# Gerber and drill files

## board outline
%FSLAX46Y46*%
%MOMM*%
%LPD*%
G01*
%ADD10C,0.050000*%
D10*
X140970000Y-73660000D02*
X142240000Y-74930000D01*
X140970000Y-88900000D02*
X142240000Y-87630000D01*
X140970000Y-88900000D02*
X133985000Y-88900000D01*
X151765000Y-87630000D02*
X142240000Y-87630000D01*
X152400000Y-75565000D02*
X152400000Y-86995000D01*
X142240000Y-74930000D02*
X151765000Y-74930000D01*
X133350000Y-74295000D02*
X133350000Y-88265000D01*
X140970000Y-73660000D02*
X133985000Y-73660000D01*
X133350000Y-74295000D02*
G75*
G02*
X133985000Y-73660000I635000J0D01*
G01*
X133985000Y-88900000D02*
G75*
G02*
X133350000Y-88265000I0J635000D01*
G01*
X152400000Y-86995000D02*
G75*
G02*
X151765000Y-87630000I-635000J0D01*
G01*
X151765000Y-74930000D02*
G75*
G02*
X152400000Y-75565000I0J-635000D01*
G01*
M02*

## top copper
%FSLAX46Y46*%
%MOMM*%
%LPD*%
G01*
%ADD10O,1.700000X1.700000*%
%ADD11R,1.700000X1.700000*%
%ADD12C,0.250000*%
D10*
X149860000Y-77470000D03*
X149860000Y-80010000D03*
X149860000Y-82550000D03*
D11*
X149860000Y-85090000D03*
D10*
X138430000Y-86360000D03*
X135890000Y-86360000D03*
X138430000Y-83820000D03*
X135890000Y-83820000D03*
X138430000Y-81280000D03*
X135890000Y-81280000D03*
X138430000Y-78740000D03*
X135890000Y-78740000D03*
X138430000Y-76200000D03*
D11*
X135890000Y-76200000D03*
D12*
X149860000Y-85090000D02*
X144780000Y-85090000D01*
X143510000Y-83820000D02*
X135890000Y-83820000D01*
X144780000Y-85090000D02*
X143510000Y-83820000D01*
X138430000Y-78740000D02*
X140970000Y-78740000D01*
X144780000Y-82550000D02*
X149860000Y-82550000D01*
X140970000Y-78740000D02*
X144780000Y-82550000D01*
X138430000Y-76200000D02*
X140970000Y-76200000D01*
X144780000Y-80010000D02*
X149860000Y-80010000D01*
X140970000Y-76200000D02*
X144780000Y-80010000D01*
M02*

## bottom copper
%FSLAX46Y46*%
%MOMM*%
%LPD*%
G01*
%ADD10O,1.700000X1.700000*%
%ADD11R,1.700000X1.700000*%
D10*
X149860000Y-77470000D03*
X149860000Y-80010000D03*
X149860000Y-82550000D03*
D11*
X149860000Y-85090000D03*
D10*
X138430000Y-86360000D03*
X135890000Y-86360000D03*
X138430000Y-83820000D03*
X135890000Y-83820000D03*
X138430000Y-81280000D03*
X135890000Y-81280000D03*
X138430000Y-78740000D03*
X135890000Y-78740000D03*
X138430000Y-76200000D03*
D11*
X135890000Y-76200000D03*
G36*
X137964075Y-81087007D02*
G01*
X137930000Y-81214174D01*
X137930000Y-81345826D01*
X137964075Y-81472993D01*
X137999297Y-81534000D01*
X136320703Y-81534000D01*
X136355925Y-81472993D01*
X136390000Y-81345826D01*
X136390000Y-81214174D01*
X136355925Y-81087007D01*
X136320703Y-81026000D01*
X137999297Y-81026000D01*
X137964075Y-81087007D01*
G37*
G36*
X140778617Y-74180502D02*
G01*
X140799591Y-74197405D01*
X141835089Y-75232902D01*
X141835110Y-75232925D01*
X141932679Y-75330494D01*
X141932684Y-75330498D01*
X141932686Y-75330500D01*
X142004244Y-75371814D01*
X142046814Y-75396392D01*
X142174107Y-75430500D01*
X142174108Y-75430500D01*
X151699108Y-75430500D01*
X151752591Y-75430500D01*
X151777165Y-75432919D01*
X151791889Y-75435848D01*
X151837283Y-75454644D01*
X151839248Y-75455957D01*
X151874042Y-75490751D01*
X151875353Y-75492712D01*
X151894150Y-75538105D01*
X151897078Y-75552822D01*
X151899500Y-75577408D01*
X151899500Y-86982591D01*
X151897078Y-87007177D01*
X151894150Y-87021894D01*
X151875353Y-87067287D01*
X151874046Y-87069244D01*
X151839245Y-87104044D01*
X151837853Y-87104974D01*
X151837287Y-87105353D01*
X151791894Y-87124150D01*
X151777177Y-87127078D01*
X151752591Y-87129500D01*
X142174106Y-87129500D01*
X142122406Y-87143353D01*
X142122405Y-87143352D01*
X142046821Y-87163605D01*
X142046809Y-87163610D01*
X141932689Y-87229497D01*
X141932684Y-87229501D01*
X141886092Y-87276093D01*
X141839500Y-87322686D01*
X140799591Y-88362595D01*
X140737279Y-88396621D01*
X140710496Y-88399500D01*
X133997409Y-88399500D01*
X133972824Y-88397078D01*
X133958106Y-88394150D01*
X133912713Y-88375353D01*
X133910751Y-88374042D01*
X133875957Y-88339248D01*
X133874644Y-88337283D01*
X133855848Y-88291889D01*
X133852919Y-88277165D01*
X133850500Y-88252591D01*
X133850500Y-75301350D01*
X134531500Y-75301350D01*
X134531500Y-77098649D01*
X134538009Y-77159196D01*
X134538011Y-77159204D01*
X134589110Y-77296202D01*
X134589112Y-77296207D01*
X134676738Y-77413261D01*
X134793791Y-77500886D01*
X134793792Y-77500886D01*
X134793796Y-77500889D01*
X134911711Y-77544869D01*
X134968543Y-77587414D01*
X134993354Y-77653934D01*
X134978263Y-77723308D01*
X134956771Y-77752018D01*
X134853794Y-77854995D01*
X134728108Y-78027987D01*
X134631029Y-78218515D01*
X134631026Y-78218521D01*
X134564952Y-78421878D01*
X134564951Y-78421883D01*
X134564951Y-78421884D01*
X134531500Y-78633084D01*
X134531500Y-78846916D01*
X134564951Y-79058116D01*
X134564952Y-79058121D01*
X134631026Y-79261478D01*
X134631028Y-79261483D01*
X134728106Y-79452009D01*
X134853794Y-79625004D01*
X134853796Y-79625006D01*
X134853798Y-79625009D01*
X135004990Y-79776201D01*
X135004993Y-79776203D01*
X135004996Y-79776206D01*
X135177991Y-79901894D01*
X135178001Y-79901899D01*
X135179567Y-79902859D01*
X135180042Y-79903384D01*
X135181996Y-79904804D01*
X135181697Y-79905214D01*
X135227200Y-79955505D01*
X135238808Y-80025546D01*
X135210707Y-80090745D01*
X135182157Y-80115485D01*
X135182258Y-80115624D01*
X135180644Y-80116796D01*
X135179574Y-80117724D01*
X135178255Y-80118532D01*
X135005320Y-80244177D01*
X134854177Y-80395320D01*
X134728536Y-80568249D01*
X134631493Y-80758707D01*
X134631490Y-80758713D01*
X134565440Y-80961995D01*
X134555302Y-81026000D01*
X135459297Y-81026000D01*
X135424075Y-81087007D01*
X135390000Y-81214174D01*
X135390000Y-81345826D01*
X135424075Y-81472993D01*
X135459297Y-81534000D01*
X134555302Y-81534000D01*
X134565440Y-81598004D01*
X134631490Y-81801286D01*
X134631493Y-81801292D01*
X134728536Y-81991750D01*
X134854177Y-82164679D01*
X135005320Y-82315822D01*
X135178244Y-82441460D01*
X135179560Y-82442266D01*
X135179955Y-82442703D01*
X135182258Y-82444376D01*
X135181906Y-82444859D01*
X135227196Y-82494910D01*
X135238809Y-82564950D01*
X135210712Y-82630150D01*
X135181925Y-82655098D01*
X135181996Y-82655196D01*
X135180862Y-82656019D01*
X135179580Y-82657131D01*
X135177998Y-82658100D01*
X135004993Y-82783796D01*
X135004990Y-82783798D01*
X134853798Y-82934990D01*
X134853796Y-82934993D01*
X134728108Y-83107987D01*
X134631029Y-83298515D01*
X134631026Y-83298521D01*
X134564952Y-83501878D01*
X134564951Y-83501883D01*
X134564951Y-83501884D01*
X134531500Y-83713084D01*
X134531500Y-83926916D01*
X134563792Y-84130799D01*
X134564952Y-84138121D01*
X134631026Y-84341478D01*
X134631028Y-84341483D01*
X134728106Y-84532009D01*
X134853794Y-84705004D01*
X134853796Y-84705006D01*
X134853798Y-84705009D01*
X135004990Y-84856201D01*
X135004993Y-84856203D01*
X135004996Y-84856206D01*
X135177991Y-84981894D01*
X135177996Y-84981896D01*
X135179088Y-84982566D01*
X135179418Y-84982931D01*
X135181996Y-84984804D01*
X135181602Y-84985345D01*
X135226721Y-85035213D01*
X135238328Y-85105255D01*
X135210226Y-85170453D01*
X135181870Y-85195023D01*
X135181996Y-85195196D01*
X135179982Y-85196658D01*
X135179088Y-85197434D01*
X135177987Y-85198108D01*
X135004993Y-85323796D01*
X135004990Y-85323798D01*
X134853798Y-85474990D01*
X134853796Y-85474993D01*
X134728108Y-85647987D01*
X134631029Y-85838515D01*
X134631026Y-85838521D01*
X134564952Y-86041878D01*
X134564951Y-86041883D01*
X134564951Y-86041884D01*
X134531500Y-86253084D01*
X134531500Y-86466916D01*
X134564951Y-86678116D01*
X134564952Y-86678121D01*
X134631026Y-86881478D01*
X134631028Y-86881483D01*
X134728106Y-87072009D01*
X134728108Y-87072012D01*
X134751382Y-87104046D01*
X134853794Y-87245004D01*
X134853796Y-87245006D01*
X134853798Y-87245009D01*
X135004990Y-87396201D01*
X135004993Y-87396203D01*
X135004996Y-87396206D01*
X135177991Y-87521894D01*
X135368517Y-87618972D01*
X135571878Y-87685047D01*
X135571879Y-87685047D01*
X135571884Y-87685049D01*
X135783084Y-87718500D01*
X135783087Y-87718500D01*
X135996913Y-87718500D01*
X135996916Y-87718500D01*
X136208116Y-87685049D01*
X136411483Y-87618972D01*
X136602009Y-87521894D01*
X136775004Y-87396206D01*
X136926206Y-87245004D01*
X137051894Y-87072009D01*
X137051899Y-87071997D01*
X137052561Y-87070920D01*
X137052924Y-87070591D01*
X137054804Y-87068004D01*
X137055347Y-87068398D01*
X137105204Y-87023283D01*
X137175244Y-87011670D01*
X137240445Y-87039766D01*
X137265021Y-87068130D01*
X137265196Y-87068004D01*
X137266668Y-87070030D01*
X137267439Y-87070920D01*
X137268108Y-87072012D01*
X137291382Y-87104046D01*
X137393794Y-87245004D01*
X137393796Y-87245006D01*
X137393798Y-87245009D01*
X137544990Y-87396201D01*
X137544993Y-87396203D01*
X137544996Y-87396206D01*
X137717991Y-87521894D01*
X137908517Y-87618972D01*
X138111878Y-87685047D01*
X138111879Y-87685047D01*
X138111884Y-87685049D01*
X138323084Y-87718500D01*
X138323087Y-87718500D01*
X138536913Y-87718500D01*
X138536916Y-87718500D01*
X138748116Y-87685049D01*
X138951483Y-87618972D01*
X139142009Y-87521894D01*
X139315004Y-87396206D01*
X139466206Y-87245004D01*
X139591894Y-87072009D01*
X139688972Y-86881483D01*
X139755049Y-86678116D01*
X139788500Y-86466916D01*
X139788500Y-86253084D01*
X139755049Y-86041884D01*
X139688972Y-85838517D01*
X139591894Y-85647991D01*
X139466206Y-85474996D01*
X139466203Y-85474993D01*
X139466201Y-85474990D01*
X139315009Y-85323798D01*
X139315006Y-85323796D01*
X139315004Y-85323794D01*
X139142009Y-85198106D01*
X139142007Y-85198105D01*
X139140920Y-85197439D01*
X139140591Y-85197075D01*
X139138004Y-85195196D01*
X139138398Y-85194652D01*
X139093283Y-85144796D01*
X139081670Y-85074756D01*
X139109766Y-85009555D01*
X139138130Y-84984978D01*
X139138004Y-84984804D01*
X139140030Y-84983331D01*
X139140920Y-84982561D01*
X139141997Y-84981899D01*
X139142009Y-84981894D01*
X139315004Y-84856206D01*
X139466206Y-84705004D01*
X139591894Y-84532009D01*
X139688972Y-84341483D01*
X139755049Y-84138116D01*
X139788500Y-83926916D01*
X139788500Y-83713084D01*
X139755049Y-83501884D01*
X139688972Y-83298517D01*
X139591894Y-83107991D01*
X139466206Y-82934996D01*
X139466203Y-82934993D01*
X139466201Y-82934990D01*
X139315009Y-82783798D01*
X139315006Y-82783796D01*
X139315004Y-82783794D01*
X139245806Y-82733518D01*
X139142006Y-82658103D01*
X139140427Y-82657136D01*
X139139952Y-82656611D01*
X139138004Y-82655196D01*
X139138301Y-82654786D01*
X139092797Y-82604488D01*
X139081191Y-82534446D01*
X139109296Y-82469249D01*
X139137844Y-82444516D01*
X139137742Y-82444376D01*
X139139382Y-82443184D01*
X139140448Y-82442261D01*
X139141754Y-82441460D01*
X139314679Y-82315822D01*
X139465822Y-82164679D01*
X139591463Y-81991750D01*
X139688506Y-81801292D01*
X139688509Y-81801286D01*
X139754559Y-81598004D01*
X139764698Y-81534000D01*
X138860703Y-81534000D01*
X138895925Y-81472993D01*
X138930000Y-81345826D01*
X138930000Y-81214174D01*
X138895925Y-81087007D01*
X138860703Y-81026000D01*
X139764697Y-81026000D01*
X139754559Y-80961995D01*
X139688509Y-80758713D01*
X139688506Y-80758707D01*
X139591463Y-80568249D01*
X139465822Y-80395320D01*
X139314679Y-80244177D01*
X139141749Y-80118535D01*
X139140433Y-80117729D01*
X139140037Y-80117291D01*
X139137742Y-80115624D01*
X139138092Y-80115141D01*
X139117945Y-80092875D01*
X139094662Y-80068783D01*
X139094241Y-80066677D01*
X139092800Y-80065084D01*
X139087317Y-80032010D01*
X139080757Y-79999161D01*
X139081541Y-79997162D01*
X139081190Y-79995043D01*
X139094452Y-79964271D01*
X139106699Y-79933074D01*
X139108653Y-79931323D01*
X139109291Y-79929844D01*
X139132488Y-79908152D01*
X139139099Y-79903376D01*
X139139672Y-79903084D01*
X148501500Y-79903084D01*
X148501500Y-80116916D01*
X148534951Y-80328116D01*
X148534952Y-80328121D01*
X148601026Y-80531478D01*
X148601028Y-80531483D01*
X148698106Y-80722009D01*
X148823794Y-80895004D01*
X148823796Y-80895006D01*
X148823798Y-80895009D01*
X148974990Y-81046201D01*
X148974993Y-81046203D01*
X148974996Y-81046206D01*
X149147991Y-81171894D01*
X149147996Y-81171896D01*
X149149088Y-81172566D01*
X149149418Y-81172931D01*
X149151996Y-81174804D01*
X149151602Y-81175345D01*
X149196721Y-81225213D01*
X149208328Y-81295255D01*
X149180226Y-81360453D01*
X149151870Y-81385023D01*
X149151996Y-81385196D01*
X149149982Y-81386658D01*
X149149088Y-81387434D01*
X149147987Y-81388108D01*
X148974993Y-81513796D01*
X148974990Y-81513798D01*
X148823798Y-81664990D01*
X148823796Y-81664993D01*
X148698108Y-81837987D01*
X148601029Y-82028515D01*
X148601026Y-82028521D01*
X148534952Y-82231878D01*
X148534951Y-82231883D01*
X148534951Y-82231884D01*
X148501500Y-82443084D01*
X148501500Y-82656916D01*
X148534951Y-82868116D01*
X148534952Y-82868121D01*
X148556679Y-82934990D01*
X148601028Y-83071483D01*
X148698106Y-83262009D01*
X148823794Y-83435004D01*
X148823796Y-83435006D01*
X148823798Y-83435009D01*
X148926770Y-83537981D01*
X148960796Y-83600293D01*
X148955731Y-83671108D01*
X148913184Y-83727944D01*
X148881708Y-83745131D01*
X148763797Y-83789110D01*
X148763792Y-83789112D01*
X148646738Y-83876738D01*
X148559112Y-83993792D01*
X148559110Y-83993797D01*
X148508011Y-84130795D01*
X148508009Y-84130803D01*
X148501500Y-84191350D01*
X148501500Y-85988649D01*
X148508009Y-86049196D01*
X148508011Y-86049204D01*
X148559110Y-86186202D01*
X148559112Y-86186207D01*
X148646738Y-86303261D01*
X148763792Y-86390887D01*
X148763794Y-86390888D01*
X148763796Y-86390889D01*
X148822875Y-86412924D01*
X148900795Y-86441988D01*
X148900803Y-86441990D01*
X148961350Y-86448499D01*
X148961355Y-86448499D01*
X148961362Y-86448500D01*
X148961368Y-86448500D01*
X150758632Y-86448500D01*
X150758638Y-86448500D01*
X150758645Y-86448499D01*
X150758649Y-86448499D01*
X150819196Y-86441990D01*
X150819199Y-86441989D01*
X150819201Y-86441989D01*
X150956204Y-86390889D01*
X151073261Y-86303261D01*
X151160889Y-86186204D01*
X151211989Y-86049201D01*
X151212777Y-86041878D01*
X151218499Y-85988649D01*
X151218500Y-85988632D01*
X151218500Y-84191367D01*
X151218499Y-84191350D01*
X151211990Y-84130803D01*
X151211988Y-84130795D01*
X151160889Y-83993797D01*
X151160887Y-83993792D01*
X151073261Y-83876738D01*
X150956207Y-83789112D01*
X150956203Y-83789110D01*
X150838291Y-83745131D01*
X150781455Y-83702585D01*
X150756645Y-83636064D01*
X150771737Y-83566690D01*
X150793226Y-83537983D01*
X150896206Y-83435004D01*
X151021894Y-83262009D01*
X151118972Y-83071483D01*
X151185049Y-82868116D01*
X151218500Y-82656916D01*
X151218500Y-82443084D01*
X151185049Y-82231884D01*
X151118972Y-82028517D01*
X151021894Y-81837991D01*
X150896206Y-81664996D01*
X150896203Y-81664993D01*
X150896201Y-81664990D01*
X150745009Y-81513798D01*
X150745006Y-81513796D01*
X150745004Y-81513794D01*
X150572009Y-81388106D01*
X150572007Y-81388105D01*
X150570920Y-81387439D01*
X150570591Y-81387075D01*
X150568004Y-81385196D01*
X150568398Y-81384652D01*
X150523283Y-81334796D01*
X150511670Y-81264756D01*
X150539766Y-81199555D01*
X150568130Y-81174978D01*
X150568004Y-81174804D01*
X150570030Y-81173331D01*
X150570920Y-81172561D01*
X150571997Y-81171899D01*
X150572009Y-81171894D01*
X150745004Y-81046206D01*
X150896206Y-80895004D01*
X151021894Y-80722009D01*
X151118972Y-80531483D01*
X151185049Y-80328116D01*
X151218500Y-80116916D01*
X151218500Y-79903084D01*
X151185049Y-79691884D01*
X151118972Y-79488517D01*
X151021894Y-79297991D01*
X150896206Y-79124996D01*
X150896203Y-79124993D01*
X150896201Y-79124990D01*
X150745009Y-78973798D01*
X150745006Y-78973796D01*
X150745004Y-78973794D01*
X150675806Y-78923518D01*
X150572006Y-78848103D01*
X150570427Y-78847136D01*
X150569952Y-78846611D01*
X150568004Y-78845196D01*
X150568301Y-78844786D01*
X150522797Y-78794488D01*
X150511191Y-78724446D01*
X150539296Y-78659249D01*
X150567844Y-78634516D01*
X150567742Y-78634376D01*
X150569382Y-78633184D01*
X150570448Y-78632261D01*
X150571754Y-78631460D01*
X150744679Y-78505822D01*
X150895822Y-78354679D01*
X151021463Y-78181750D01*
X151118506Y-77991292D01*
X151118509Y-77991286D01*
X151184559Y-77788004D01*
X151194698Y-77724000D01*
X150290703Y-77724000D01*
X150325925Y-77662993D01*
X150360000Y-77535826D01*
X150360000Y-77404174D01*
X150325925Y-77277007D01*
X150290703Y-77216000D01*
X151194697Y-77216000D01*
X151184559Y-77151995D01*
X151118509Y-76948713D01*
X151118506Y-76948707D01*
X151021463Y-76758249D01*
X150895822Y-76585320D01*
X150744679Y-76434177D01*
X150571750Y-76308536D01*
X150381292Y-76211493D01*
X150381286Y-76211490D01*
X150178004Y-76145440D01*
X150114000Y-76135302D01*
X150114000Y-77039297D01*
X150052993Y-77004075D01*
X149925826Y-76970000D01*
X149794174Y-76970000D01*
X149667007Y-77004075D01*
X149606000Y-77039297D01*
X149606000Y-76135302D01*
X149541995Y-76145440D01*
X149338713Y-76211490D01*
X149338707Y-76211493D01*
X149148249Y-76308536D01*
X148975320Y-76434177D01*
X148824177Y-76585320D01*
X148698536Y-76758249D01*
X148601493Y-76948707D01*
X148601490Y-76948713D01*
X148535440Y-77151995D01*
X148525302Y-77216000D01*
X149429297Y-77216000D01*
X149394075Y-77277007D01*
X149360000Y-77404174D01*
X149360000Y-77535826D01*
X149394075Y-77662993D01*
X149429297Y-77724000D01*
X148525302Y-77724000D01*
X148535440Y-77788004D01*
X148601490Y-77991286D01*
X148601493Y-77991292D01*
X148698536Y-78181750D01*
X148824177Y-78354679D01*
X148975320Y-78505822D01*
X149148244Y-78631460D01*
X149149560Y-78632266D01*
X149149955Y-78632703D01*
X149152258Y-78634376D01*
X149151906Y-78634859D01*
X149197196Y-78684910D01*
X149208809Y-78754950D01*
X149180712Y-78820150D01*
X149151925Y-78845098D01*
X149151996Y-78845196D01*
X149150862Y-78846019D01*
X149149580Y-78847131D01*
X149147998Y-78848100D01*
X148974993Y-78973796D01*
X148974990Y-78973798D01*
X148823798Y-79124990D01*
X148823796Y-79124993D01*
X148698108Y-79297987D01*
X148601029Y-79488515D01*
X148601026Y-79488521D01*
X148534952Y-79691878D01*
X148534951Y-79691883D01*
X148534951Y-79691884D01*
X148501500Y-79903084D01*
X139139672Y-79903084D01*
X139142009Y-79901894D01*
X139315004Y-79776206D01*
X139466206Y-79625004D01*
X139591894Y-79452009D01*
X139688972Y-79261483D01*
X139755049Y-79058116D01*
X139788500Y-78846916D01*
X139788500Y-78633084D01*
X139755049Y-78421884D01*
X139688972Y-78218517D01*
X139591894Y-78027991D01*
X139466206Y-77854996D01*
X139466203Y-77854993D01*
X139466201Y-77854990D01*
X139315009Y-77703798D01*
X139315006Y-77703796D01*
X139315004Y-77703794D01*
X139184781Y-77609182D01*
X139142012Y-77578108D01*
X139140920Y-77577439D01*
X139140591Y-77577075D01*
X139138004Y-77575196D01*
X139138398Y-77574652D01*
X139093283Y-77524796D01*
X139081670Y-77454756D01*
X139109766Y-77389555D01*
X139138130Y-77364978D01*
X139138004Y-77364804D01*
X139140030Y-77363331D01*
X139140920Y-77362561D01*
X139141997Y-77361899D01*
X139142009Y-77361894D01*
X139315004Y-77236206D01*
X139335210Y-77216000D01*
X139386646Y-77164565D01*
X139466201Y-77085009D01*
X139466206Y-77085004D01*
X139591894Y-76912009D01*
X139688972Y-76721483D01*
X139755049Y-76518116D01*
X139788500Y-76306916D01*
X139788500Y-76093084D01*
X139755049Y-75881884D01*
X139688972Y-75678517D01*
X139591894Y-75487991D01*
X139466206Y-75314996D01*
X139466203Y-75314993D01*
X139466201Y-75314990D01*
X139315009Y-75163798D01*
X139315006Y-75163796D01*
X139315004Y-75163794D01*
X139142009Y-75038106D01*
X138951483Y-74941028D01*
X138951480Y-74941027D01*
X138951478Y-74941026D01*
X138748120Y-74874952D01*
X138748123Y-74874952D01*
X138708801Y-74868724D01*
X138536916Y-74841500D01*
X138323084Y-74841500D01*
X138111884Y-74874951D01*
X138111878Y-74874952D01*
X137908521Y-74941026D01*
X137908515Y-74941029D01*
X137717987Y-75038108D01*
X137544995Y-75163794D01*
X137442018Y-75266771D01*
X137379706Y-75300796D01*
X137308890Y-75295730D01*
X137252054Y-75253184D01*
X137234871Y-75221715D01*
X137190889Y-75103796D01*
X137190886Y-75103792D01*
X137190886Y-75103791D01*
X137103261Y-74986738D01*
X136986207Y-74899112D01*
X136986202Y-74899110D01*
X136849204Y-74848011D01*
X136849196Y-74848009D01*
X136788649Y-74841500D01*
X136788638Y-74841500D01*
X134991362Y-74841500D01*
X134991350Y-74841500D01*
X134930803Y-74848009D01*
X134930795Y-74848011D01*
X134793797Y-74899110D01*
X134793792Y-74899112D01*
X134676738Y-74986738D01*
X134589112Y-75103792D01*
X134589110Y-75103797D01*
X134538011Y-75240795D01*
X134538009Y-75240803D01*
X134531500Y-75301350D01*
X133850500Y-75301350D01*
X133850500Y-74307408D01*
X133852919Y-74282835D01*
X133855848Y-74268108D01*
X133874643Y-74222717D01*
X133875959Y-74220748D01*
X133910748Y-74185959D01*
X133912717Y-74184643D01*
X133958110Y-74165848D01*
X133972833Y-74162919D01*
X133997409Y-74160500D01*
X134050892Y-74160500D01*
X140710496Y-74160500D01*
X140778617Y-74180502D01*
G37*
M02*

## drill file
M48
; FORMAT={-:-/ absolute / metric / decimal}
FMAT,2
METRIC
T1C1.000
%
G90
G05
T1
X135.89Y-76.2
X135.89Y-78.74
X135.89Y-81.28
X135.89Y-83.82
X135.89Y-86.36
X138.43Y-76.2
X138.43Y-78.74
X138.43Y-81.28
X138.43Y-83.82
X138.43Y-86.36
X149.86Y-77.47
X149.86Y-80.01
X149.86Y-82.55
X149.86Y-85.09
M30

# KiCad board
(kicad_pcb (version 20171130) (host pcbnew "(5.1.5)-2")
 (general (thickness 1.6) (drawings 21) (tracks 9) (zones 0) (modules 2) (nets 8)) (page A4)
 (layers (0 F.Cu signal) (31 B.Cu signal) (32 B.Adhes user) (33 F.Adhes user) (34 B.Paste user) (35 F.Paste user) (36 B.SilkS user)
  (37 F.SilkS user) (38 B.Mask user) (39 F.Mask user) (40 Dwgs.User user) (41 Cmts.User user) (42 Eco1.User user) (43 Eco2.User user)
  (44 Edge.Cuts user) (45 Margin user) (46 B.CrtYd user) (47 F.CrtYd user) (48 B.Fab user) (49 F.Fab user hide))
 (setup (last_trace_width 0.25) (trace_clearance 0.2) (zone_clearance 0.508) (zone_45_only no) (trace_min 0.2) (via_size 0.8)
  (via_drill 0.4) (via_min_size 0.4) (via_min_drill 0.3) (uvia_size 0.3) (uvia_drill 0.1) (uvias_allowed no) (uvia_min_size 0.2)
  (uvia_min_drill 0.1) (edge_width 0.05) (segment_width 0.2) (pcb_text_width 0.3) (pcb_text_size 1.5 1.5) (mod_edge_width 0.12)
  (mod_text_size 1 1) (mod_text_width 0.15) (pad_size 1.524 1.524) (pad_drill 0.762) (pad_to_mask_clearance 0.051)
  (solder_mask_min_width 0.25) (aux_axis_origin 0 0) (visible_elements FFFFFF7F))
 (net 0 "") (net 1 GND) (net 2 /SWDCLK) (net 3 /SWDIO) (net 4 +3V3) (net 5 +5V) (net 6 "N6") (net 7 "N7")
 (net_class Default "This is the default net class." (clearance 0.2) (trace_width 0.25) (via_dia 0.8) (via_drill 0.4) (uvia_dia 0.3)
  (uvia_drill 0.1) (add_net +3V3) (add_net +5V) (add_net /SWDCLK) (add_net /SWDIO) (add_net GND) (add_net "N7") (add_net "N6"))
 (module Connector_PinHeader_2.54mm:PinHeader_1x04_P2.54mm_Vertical (layer F.Cu) (at 149.86 85.09 180)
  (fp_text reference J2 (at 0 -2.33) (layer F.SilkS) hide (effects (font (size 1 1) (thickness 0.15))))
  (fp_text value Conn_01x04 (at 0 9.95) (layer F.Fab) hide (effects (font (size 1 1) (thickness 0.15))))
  (pad 4 thru_hole oval (at 0 7.62 180) (size 1.7 1.7) (drill 1) (layers *.Cu *.Mask) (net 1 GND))
  (pad 3 thru_hole oval (at 0 5.08 180) (size 1.7 1.7) (drill 1) (layers *.Cu *.Mask) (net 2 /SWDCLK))
  (pad 2 thru_hole oval (at 0 2.54 180) (size 1.7 1.7) (drill 1) (layers *.Cu *.Mask) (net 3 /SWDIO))
  (pad 1 thru_hole rect (at 0 0 180) (size 1.7 1.7) (drill 1) (layers *.Cu *.Mask) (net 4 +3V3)))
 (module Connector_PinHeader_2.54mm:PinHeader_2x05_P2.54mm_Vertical (layer F.Cu) (at 135.89 76.2)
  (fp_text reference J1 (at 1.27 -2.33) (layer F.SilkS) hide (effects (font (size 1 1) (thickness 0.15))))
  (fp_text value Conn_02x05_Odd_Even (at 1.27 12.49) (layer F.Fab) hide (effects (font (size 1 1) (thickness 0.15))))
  (pad 10 thru_hole oval (at 2.54 10.16) (size 1.7 1.7) (drill 1) (layers *.Cu *.Mask) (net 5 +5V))
  (pad 9 thru_hole oval (at 0 10.16) (size 1.7 1.7) (drill 1) (layers *.Cu *.Mask) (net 5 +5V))
  (pad 8 thru_hole oval (at 2.54 7.62) (size 1.7 1.7) (drill 1) (layers *.Cu *.Mask) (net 4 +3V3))
  (pad 7 thru_hole oval (at 0 7.62) (size 1.7 1.7) (drill 1) (layers *.Cu *.Mask) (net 4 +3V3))
  (pad 6 thru_hole oval (at 2.54 5.08) (size 1.7 1.7) (drill 1) (layers *.Cu *.Mask) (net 1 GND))
  (pad 5 thru_hole oval (at 0 5.08) (size 1.7 1.7) (drill 1) (layers *.Cu *.Mask) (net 1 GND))
  (pad 4 thru_hole oval (at 2.54 2.54) (size 1.7 1.7) (drill 1) (layers *.Cu *.Mask) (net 3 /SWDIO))
  (pad 3 thru_hole oval (at 0 2.54) (size 1.7 1.7) (drill 1) (layers *.Cu *.Mask) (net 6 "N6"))
  (pad 2 thru_hole oval (at 2.54 0) (size 1.7 1.7) (drill 1) (layers *.Cu *.Mask) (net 2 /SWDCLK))
  (pad 1 thru_hole rect (at 0 0) (size 1.7 1.7) (drill 1) (layers *.Cu *.Mask) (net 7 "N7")))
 (gr_line (start 140.97 73.66) (end 142.24 74.93) (layer Edge.Cuts) (width 0.05))
 (gr_line (start 140.97 88.9) (end 142.24 87.63) (layer Edge.Cuts) (width 0.05))
 (gr_line (start 140.97 88.9) (end 133.985 88.9) (layer Edge.Cuts) (width 0.05))
 (gr_line (start 151.765 87.63) (end 142.24 87.63) (layer Edge.Cuts) (width 0.05))
 (gr_line (start 152.4 75.565) (end 152.4 86.995) (layer Edge.Cuts) (width 0.05))
 (gr_line (start 142.24 74.93) (end 151.765 74.93) (layer Edge.Cuts) (width 0.05))
 (gr_line (start 133.35 74.295) (end 133.35 88.265) (layer Edge.Cuts) (width 0.05))
 (gr_line (start 140.97 73.66) (end 133.985 73.66) (layer Edge.Cuts) (width 0.05))
 (gr_arc (start 133.985 74.295) (end 133.985 73.66) (angle -90) (layer Edge.Cuts) (width 0.05))
 (gr_arc (start 133.985 88.265) (end 133.35 88.265) (angle -90) (layer Edge.Cuts) (width 0.05))
 (gr_arc (start 151.765 86.995) (end 151.765 87.63) (angle -90) (layer Edge.Cuts) (width 0.05))
 (gr_arc (start 151.765 75.565) (end 152.4 75.565) (angle -90) (layer Edge.Cuts) (width 0.05))
 (segment (start 149.86 85.09) (end 144.78 85.09) (width 0.25) (layer F.Cu) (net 4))
 (segment (start 143.51 83.82) (end 135.89 83.82) (width 0.25) (layer F.Cu) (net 4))
 (segment (start 144.78 85.09) (end 143.51 83.82) (width 0.25) (layer F.Cu) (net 4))
 (segment (start 138.43 78.74) (end 140.97 78.74) (width 0.25) (layer F.Cu) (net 3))
 (segment (start 144.78 82.55) (end 149.86 82.55) (width 0.25) (layer F.Cu) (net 3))
 (segment (start 140.97 78.74) (end 144.78 82.55) (width 0.25) (layer F.Cu) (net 3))
 (segment (start 138.43 76.2) (end 140.97 76.2) (width 0.25) (layer F.Cu) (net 2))
 (segment (start 144.78 80.01) (end 149.86 80.01) (width 0.25) (layer F.Cu) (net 2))
 (segment (start 140.97 76.2) (end 144.78 80.01) (width 0.25) (layer F.Cu) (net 2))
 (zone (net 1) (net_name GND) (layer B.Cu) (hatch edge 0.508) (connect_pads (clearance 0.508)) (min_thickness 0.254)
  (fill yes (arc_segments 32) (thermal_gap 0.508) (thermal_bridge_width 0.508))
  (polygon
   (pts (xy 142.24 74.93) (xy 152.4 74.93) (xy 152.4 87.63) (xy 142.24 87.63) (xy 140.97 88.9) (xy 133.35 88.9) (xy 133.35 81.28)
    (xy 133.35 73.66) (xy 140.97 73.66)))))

